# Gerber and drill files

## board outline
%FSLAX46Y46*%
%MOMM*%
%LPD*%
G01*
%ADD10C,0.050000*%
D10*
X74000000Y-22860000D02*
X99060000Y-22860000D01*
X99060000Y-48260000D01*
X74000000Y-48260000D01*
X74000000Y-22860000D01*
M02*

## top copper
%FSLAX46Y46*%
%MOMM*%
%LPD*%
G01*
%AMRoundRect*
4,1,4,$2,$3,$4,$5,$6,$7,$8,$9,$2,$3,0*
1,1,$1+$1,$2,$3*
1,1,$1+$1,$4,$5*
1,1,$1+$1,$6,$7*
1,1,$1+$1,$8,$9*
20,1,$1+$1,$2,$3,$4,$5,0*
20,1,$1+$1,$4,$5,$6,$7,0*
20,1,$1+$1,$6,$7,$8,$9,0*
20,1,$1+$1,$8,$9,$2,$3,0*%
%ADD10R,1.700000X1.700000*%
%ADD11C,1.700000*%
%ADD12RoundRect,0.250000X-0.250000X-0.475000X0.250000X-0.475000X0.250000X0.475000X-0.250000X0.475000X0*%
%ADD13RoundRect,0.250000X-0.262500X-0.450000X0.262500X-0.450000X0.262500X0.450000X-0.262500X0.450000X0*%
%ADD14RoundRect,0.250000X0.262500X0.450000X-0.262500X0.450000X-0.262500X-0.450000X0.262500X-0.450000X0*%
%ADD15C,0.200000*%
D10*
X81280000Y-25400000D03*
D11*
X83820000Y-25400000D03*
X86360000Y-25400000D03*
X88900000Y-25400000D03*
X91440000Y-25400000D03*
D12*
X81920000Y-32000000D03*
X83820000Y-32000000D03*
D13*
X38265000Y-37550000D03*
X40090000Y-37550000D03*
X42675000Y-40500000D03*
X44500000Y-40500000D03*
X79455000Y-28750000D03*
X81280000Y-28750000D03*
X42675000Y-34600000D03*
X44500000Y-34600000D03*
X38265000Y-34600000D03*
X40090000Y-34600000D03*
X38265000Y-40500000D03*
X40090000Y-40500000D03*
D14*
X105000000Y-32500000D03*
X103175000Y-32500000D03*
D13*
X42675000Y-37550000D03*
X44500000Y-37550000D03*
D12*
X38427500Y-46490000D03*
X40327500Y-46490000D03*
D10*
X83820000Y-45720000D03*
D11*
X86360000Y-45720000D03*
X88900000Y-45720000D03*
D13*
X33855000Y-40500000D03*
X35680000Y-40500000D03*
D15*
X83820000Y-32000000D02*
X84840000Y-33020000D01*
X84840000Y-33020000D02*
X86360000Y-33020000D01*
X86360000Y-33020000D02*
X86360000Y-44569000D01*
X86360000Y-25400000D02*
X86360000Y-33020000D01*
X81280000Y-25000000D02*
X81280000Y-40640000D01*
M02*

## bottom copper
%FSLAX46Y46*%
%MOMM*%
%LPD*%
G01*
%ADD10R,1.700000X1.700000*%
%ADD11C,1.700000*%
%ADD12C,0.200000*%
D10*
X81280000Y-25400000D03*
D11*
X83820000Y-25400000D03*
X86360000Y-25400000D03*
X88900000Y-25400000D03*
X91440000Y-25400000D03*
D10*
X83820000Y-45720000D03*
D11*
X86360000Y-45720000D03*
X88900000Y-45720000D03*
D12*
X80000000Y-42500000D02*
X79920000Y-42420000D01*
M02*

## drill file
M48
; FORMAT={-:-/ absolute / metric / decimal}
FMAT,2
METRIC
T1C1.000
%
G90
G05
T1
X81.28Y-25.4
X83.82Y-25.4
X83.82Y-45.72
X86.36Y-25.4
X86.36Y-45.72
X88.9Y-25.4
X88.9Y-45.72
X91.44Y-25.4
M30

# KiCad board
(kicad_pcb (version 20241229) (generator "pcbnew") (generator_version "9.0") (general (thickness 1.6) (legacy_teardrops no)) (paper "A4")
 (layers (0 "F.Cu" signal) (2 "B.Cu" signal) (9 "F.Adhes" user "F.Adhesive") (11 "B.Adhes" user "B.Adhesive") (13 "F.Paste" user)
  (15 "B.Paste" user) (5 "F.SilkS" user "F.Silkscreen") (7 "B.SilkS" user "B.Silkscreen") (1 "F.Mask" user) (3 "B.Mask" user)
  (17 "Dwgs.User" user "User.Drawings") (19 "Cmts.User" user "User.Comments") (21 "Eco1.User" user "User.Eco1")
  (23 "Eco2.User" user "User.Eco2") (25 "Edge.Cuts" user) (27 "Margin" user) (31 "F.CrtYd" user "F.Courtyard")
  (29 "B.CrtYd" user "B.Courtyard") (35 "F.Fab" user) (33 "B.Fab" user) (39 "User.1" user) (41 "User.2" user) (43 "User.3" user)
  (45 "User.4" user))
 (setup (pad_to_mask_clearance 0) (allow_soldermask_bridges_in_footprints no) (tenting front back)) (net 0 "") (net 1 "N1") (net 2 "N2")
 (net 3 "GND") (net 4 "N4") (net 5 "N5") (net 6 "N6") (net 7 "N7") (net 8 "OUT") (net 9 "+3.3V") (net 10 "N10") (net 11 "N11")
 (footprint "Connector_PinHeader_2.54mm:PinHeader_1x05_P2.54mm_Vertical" (layer "F.Cu") (at 81.28 25.4 90)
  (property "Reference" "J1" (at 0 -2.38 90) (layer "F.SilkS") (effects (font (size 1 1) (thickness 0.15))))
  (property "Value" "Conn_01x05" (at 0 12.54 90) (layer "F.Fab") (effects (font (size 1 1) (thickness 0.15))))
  (pad "1" thru_hole rect (at 0 0 90) (size 1.7 1.7) (drill 1) (layers "*.Cu" "*.Mask") (remove_unused_layers no) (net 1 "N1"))
  (pad "2" thru_hole circle (at 0 2.54 90) (size 1.7 1.7) (drill 1) (layers "*.Cu" "*.Mask") (remove_unused_layers no) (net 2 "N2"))
  (pad "3" thru_hole circle (at 0 5.08 90) (size 1.7 1.7) (drill 1) (layers "*.Cu" "*.Mask") (remove_unused_layers no) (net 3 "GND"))
  (pad "4" thru_hole circle (at 0 7.62 90) (size 1.7 1.7) (drill 1) (layers "*.Cu" "*.Mask") (remove_unused_layers no) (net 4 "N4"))
  (pad "5" thru_hole circle (at 0 10.16 90) (size 1.7 1.7) (drill 1) (layers "*.Cu" "*.Mask") (remove_unused_layers no) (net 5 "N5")))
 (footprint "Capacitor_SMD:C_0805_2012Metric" (layer "F.Cu") (at 82.87 32)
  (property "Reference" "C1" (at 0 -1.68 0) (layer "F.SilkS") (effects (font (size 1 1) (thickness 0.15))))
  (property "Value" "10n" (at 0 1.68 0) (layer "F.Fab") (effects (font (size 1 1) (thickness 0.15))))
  (pad "1" smd roundrect (at -0.95 0) (size 1 1.45) (layers "F.Cu" "F.Mask" "F.Paste") (roundrect_rratio 0.25) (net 1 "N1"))
  (pad "2" smd roundrect (at 0.95 0) (size 1 1.45) (layers "F.Cu" "F.Mask" "F.Paste") (roundrect_rratio 0.25) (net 3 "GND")))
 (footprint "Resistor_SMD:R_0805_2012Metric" (layer "F.Cu") (at 39.1775 37.55)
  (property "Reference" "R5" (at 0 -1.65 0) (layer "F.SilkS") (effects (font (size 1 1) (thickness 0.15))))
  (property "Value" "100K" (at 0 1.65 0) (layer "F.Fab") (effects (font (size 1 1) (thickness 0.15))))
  (pad "1" smd roundrect (at -0.9125 0) (size 1.025 1.4) (layers "F.Cu" "F.Mask" "F.Paste") (roundrect_rratio 0.243902) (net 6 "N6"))
  (pad "2" smd roundrect (at 0.9125 0) (size 1.025 1.4) (layers "F.Cu" "F.Mask" "F.Paste") (roundrect_rratio 0.243902) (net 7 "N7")))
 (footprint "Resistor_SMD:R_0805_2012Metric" (layer "F.Cu") (at 43.5875 40.5)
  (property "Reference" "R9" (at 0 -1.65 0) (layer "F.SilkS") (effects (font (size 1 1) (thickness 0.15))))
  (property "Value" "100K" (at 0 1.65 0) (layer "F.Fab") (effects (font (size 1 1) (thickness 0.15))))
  (pad "1" smd roundrect (at -0.9125 0) (size 1.025 1.4) (layers "F.Cu" "F.Mask" "F.Paste") (roundrect_rratio 0.243902) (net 7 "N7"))
  (pad "2" smd roundrect (at 0.9125 0) (size 1.025 1.4) (layers "F.Cu" "F.Mask" "F.Paste") (roundrect_rratio 0.243902) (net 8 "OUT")))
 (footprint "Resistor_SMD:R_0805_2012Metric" (layer "F.Cu") (at 80.3675 28.75)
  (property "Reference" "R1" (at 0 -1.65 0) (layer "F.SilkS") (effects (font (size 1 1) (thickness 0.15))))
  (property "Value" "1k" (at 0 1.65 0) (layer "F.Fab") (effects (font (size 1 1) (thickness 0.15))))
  (pad "1" smd roundrect (at -0.9125 0) (size 1.025 1.4) (layers "F.Cu" "F.Mask" "F.Paste") (roundrect_rratio 0.243902) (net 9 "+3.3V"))
  (pad "2" smd roundrect (at 0.9125 0) (size 1.025 1.4) (layers "F.Cu" "F.Mask" "F.Paste") (roundrect_rratio 0.243902) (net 1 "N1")))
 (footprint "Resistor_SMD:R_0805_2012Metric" (layer "F.Cu") (at 43.5875 34.6)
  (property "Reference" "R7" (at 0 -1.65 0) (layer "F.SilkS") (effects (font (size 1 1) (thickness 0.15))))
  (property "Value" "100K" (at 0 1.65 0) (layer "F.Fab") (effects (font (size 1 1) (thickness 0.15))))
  (pad "1" smd roundrect (at -0.9125 0) (size 1.025 1.4) (layers "F.Cu" "F.Mask" "F.Paste") (roundrect_rratio 0.243902) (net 3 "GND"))
  (pad "2" smd roundrect (at 0.9125 0) (size 1.025 1.4) (layers "F.Cu" "F.Mask" "F.Paste") (roundrect_rratio 0.243902) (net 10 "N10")))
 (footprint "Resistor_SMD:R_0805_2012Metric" (layer "F.Cu") (at 39.1775 34.6)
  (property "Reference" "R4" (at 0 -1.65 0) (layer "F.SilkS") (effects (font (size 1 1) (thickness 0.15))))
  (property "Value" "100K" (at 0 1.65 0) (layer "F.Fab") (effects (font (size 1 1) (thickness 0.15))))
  (pad "1" smd roundrect (at -0.9125 0) (size 1.025 1.4) (layers "F.Cu" "F.Mask" "F.Paste") (roundrect_rratio 0.243902) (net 5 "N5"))
  (pad "2" smd roundrect (at 0.9125 0) (size 1.025 1.4) (layers "F.Cu" "F.Mask" "F.Paste") (roundrect_rratio 0.243902) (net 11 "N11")))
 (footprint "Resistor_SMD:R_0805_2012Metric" (layer "F.Cu") (at 39.1775 40.5)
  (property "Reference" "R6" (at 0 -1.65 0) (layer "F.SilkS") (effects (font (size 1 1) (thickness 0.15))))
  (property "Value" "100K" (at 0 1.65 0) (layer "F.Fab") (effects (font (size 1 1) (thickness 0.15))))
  (pad "1" smd roundrect (at -0.9125 0) (size 1.025 1.4) (layers "F.Cu" "F.Mask" "F.Paste") (roundrect_rratio 0.243902) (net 11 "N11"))
  (pad "2" smd roundrect (at 0.9125 0) (size 1.025 1.4) (layers "F.Cu" "F.Mask" "F.Paste") (roundrect_rratio 0.243902) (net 8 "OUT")))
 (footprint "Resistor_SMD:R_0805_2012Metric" (layer "F.Cu") (at 104.0875 32.5 180)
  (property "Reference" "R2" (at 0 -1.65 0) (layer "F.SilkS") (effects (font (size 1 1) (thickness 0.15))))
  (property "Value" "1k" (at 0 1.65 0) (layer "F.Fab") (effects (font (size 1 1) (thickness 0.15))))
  (pad "1" smd roundrect (at -0.9125 0 180) (size 1.025 1.4) (layers "F.Cu" "F.Mask" "F.Paste") (roundrect_rratio 0.243902) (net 9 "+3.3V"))
  (pad "2" smd roundrect (at 0.9125 0 180) (size 1.025 1.4) (layers "F.Cu" "F.Mask" "F.Paste") (roundrect_rratio 0.243902) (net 5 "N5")))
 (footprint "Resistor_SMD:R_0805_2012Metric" (layer "F.Cu") (at 43.5875 37.55)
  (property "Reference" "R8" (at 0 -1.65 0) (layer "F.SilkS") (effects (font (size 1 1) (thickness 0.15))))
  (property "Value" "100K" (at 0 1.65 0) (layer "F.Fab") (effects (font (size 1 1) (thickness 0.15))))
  (pad "1" smd roundrect (at -0.9125 0) (size 1.025 1.4) (layers "F.Cu" "F.Mask" "F.Paste") (roundrect_rratio 0.243902) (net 10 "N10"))
  (pad "2" smd roundrect (at 0.9125 0) (size 1.025 1.4) (layers "F.Cu" "F.Mask" "F.Paste") (roundrect_rratio 0.243902) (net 7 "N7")))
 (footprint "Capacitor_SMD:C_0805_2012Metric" (layer "F.Cu") (at 39.3775 46.49)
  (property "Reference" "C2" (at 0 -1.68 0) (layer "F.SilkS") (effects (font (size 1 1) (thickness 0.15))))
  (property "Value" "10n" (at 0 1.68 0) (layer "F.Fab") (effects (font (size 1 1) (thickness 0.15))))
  (pad "1" smd roundrect (at -0.95 0) (size 1 1.45) (layers "F.Cu" "F.Mask" "F.Paste") (roundrect_rratio 0.25) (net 5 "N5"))
  (pad "2" smd roundrect (at 0.95 0) (size 1 1.45) (layers "F.Cu" "F.Mask" "F.Paste") (roundrect_rratio 0.25) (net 3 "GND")))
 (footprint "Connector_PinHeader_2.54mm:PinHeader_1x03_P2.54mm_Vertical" (layer "F.Cu") (at 83.82 45.72 90)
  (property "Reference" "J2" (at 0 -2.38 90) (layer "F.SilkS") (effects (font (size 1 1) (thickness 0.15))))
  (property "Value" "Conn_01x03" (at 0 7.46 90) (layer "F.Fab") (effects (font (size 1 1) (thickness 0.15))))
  (pad "1" thru_hole rect (at 0 0 90) (size 1.7 1.7) (drill 1) (layers "*.Cu" "*.Mask") (remove_unused_layers no) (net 9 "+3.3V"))
  (pad "2" thru_hole circle (at 0 2.54 90) (size 1.7 1.7) (drill 1) (layers "*.Cu" "*.Mask") (remove_unused_layers no) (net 8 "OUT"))
  (pad "3" thru_hole circle (at 0 5.08 90) (size 1.7 1.7) (drill 1) (layers "*.Cu" "*.Mask") (remove_unused_layers no) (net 3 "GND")))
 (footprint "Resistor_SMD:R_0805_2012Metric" (layer "F.Cu") (at 34.7675 40.5)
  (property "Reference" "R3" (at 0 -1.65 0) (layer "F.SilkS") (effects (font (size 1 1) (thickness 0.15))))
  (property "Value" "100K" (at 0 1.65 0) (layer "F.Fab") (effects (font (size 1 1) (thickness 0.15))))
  (pad "1" smd roundrect (at -0.9125 0) (size 1.025 1.4) (layers "F.Cu" "F.Mask" "F.Paste") (roundrect_rratio 0.243902) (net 1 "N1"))
  (pad "2" smd roundrect (at 0.9125 0) (size 1.025 1.4) (layers "F.Cu" "F.Mask" "F.Paste") (roundrect_rratio 0.243902) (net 6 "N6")))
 (gr_rect (start 74 22.86) (end 99.06 48.26) (stroke (width 0.05) (type default)) (fill no) (layer "Edge.Cuts"))
 (segment (start 83.82 32) (end 84.84 33.02) (width 0.2) (layer "F.Cu") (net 3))
 (segment (start 84.84 33.02) (end 86.36 33.02) (width 0.2) (layer "F.Cu") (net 3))
 (segment (start 86.36 33.02) (end 86.36 44.569) (width 0.2) (layer "F.Cu") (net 3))
 (segment (start 86.36 25.4) (end 86.36 33.02) (width 0.2) (layer "F.Cu") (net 3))
 (segment (start 81.28 25) (end 81.28 40.64) (width 0.2) (layer "F.Cu") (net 1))
 (segment (start 80 42.5) (end 79.92 42.42) (width 0.2) (layer "B.Cu") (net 1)))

